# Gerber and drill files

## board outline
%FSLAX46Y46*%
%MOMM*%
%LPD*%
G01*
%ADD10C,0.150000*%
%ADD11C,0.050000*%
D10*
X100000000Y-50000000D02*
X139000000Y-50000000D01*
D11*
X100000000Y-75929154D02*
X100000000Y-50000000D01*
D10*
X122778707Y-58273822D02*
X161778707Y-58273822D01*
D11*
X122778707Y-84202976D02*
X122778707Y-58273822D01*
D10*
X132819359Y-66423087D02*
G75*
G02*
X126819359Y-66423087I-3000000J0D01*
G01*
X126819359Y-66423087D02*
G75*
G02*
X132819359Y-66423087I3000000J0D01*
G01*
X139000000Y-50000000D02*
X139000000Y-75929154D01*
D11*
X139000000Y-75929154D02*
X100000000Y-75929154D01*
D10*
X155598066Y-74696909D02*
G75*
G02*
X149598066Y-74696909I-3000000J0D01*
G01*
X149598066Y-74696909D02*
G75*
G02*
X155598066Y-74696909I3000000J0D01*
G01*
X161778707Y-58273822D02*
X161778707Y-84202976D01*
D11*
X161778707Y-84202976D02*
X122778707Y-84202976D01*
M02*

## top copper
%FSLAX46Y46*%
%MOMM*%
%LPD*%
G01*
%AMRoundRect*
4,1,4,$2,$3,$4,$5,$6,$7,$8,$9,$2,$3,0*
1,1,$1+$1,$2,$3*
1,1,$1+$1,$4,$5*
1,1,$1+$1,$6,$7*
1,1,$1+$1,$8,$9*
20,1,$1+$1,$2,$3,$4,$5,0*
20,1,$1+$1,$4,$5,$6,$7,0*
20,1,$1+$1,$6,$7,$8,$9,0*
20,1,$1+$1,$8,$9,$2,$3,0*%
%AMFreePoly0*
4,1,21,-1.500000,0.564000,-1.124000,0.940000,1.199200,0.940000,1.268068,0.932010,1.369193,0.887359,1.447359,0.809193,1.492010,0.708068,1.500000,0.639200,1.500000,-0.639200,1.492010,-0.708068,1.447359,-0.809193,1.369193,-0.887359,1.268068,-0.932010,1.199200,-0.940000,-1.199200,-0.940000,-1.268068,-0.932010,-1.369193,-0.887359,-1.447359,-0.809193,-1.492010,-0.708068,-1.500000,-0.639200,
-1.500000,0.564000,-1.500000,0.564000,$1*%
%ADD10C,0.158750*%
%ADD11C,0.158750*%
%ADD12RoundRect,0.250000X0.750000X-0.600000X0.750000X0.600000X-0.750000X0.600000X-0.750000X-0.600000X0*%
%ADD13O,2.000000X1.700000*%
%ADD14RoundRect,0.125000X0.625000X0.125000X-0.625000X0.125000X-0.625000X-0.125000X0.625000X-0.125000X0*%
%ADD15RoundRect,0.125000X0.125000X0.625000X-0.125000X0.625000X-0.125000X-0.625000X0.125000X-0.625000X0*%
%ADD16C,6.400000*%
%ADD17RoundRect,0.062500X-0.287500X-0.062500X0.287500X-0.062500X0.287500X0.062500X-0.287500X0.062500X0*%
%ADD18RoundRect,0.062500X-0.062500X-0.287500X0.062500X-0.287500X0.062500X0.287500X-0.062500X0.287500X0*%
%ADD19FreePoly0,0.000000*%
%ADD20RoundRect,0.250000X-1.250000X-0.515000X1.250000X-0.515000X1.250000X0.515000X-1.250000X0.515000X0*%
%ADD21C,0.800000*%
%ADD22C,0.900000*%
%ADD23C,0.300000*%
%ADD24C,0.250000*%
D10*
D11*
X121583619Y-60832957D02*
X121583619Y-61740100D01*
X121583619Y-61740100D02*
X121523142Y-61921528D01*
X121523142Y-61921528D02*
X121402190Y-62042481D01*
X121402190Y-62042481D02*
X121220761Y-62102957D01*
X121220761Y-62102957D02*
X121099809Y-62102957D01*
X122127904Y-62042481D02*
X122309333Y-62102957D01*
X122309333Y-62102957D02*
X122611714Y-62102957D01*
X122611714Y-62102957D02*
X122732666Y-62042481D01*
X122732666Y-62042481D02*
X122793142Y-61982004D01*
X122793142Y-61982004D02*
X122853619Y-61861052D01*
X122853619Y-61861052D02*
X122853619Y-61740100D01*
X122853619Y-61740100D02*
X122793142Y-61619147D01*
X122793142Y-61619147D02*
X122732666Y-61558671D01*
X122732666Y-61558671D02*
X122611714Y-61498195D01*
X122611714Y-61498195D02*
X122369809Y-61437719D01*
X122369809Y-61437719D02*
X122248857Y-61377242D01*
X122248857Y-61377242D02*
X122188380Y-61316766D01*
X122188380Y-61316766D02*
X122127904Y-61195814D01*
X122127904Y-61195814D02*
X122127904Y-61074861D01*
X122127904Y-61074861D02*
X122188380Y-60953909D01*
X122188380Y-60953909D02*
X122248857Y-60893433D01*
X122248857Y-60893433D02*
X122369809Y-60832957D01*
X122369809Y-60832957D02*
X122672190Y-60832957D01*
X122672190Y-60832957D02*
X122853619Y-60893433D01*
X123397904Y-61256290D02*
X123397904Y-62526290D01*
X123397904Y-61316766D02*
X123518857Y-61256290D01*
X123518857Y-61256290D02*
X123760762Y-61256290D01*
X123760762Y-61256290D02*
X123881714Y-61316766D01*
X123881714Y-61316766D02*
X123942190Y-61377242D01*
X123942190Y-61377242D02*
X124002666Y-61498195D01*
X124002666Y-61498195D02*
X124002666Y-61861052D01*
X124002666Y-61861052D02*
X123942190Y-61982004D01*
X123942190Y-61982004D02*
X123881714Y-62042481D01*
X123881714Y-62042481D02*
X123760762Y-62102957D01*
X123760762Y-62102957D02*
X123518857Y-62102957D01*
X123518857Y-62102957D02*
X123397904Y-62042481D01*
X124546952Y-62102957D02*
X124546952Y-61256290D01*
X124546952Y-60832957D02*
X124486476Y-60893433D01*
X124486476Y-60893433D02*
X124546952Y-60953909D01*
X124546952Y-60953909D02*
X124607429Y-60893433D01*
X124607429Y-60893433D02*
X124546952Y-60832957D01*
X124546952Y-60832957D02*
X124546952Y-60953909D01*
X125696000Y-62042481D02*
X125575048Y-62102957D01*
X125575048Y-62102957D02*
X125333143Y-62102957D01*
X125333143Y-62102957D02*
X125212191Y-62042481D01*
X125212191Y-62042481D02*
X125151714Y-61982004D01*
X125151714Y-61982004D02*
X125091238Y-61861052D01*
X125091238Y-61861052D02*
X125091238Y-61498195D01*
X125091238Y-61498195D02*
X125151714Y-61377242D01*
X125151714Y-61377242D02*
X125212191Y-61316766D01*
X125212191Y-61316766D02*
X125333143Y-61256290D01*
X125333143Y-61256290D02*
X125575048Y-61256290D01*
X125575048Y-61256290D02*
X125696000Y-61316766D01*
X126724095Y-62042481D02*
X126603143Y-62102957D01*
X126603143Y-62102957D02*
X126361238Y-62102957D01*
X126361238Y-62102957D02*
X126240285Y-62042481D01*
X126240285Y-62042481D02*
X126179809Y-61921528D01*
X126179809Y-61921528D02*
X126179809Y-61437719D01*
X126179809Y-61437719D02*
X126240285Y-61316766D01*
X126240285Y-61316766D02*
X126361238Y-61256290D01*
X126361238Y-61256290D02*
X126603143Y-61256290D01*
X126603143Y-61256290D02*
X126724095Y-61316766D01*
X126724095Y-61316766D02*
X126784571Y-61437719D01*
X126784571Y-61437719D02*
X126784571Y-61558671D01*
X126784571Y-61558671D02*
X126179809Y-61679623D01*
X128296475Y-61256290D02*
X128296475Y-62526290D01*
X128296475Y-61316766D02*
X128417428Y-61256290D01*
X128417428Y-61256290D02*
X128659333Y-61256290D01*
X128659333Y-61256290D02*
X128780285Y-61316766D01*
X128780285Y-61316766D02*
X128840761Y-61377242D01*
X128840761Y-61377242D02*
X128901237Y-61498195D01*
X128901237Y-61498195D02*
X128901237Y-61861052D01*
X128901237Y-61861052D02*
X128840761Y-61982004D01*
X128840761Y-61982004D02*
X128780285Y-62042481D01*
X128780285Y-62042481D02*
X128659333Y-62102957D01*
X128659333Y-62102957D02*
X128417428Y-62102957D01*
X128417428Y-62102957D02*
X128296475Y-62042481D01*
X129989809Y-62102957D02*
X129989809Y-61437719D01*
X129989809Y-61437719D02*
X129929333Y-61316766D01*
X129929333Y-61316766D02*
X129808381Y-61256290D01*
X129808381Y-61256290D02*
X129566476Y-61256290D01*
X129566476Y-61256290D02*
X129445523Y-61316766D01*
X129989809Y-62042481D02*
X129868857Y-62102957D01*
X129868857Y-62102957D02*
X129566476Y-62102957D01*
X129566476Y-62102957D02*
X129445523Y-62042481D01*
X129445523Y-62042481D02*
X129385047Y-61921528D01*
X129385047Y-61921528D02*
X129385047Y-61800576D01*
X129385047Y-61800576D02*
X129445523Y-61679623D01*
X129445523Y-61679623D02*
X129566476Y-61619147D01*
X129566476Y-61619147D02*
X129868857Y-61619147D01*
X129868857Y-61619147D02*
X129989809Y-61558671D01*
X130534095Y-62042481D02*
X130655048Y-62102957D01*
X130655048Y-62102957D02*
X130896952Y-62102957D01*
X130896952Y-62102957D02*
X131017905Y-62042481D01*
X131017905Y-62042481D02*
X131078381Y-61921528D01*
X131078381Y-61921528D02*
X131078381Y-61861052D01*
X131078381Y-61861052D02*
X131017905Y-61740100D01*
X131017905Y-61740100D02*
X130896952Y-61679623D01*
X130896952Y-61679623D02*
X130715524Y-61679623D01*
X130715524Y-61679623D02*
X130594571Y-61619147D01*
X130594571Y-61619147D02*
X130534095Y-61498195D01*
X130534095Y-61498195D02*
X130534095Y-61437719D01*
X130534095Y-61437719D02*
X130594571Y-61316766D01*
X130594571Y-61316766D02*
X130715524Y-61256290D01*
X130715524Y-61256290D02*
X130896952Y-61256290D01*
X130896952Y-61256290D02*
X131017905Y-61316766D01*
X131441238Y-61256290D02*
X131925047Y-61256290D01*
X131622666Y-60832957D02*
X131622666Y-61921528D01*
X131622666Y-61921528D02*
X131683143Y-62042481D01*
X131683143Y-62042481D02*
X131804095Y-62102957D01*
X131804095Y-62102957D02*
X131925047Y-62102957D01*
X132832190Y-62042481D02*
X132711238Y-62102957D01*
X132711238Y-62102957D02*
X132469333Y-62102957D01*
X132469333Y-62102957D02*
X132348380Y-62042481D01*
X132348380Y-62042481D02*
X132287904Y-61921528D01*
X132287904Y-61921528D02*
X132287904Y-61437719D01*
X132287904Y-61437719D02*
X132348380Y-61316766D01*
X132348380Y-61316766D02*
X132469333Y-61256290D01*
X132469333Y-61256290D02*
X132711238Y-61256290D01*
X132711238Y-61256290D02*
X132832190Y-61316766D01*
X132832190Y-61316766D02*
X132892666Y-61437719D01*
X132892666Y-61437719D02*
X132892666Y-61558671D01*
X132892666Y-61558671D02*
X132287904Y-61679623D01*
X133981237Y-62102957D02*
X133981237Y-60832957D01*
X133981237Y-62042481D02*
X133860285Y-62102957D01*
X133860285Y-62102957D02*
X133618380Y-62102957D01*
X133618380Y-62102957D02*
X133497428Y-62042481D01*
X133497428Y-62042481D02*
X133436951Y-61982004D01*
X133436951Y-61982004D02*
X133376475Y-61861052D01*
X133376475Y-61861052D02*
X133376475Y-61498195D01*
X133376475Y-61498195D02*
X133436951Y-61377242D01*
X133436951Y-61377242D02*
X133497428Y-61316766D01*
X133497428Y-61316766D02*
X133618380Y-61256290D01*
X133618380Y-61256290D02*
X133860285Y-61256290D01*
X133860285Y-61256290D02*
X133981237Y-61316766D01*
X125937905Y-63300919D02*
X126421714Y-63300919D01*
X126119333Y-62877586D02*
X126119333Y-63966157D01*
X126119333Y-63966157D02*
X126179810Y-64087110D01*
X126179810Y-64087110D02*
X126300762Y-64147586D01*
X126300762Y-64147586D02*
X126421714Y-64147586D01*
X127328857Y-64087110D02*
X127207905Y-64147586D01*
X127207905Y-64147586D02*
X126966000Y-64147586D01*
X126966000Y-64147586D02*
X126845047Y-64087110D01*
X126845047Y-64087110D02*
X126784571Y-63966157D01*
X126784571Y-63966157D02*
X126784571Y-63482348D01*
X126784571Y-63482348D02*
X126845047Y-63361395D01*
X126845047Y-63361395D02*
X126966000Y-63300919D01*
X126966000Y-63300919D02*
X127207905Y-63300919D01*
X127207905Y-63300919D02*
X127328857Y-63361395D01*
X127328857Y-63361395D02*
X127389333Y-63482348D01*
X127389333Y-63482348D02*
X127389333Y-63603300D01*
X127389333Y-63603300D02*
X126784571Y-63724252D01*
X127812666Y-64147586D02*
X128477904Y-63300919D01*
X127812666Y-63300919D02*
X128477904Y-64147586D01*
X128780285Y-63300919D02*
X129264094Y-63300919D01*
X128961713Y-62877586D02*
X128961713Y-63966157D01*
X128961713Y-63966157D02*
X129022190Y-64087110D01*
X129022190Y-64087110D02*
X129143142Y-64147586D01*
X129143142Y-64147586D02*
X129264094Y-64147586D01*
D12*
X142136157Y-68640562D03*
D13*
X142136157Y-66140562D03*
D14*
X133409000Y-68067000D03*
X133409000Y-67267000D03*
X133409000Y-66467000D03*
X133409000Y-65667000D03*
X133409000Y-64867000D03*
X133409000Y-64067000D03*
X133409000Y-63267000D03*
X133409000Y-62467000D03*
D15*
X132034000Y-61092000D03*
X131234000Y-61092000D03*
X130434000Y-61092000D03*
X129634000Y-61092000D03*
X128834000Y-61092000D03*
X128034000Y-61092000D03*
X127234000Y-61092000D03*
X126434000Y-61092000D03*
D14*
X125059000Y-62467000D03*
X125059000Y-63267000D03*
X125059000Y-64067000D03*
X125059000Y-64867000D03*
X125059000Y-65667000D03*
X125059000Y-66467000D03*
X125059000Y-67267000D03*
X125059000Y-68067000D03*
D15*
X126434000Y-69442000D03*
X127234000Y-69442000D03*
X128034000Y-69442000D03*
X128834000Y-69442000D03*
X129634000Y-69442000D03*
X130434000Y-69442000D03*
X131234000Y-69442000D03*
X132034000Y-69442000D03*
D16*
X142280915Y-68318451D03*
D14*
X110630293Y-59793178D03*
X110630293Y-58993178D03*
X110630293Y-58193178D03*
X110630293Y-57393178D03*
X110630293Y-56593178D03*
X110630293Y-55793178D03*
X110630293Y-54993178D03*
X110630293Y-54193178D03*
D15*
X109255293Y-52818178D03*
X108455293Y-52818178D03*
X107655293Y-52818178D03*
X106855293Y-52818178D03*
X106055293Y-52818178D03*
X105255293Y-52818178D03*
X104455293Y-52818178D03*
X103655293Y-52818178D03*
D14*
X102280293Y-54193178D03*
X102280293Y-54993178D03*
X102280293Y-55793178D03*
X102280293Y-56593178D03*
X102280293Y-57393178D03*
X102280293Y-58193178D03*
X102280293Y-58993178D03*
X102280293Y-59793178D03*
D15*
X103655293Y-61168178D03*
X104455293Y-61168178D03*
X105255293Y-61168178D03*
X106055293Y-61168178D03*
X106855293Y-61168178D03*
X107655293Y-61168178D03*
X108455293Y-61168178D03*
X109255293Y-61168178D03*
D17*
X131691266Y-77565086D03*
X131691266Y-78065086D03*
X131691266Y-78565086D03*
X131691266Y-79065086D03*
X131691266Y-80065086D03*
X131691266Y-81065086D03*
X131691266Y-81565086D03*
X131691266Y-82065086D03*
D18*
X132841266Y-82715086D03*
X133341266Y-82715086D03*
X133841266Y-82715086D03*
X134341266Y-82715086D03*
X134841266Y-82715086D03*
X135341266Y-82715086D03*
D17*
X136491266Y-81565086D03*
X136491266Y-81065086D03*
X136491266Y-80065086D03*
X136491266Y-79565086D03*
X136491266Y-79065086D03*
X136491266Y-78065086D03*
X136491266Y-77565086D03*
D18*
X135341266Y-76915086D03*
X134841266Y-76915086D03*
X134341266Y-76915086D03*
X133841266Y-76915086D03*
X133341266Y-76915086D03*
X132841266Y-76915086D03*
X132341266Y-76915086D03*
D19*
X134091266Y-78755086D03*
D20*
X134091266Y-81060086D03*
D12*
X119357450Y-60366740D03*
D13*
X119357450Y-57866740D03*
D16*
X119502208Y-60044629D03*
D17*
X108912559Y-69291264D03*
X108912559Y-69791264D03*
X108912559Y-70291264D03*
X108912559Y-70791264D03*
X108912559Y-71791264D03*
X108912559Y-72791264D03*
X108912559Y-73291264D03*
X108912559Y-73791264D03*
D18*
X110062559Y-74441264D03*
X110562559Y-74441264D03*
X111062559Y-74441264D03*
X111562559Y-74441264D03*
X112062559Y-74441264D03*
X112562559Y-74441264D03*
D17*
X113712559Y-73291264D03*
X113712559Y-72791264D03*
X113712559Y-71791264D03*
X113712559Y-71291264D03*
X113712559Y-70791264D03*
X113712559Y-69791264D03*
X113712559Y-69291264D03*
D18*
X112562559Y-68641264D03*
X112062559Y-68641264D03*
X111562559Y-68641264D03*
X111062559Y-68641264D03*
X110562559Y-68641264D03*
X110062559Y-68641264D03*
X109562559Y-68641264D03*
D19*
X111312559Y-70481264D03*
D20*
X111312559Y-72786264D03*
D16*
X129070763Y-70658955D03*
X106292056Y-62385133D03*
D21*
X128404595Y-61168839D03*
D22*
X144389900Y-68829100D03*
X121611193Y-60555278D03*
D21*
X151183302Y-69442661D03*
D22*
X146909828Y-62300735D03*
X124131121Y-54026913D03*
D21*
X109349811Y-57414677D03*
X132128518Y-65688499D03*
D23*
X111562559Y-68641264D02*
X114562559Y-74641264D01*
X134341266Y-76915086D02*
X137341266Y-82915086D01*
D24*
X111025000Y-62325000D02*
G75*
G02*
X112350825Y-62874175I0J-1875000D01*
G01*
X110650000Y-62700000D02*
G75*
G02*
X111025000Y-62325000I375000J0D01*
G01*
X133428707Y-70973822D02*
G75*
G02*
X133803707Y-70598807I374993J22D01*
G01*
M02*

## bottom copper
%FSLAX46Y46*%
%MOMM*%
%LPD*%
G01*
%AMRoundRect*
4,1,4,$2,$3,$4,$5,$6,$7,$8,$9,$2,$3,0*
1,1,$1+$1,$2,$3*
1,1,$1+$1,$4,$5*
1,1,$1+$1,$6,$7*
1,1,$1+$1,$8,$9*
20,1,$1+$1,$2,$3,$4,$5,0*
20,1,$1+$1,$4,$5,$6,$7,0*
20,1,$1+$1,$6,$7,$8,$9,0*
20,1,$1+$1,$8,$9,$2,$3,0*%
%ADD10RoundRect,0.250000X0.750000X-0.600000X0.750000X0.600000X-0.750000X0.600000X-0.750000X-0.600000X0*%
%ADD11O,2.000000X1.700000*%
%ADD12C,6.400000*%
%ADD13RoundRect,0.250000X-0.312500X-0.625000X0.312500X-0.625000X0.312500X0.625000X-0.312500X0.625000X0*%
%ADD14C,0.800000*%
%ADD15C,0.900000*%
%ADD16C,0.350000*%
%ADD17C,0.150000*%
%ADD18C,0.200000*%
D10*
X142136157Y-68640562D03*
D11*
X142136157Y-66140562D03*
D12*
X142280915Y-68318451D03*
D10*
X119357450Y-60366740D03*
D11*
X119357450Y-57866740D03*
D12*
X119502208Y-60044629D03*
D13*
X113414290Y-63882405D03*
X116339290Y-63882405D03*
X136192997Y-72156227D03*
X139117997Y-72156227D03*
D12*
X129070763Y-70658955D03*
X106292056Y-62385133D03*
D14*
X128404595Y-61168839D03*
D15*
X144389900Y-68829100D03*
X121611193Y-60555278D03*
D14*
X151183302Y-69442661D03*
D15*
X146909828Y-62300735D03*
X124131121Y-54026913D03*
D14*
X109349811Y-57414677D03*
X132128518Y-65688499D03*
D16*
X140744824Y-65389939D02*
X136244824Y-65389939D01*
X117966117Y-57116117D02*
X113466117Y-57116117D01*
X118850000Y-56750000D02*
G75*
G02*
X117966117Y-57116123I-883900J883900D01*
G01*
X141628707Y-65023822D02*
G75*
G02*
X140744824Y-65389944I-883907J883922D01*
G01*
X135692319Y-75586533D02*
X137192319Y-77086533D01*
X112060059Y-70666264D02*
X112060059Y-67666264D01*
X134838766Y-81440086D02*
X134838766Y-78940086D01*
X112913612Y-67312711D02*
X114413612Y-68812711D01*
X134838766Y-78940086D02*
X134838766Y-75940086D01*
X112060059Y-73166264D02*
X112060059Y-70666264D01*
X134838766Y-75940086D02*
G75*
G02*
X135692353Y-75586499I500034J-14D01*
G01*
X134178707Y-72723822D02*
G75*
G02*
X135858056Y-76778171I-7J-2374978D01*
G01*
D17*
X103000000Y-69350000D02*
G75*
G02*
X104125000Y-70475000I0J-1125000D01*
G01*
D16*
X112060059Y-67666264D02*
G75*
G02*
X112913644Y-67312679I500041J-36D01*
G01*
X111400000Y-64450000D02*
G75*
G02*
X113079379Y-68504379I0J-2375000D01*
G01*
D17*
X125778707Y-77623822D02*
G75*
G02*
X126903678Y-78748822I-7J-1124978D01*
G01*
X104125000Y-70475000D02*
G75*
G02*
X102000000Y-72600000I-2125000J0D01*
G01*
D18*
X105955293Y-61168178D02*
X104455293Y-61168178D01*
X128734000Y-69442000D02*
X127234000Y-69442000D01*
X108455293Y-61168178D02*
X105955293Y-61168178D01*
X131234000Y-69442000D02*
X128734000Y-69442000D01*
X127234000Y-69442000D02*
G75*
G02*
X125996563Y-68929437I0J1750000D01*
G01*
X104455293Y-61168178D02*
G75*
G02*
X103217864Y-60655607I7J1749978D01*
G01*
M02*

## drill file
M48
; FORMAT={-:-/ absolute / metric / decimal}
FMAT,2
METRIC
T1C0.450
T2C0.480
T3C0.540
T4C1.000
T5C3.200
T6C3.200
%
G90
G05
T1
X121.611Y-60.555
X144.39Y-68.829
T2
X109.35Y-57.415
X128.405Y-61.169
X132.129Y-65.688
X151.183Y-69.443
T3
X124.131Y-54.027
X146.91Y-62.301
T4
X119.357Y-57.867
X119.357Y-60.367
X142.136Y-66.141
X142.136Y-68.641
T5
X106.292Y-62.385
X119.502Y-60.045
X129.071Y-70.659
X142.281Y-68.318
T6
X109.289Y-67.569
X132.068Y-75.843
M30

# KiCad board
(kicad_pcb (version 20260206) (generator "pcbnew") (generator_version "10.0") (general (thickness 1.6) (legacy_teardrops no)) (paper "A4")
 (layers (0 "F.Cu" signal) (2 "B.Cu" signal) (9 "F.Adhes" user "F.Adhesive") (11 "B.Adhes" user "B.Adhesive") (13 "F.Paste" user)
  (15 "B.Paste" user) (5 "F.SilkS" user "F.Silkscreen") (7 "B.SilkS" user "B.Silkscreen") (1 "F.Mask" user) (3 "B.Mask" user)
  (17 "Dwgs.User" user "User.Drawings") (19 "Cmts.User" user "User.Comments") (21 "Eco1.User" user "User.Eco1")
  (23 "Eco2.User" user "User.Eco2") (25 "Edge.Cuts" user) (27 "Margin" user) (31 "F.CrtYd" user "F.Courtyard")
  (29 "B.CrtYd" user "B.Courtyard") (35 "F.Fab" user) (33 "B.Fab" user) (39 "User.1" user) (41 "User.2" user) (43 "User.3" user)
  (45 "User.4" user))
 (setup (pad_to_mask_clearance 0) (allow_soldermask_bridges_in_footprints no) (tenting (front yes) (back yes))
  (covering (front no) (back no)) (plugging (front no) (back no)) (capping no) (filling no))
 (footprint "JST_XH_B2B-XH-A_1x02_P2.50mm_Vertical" (layer "F.Cu") (at 142.136157 68.640562 90)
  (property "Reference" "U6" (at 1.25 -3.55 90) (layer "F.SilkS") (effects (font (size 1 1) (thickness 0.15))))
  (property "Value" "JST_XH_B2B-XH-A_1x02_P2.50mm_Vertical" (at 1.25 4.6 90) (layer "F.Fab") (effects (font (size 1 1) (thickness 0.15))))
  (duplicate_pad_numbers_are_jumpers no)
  (pad "1" thru_hole roundrect (at 0 0 90) (size 1.7 2) (drill 1) (layers "*.Cu" "*.Mask") (remove_unused_layers no)
   (roundrect_rratio 0.147059) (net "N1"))
  (pad "2" thru_hole oval (at 2.5 0 90) (size 1.7 2) (drill 1) (layers "*.Cu" "*.Mask") (remove_unused_layers no)))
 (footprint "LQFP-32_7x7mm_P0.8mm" (layer "F.Cu") (at 129.234 65.267 180)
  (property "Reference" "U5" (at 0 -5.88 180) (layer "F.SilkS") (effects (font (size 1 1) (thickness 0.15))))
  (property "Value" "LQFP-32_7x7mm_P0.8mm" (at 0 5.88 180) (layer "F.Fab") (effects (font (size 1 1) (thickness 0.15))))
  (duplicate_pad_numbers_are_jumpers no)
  (pad "1" smd roundrect (at -4.175 -2.8 180) (size 1.5 0.5) (layers "F.Cu" "F.Mask" "F.Paste") (roundrect_rratio 0.25) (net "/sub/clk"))
  (pad "2" smd roundrect (at -4.175 -2 180) (size 1.5 0.5) (layers "F.Cu" "F.Mask" "F.Paste") (roundrect_rratio 0.25) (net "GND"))
  (pad "3" smd roundrect (at -4.175 -1.2 180) (size 1.5 0.5) (layers "F.Cu" "F.Mask" "F.Paste") (roundrect_rratio 0.25) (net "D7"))
  (pad "4" smd roundrect (at -4.175 -0.4 180) (size 1.5 0.5) (layers "F.Cu" "F.Mask" "F.Paste") (roundrect_rratio 0.25) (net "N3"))
  (pad "5" smd roundrect (at -4.175 0.4 180) (size 1.5 0.5) (layers "F.Cu" "F.Mask" "F.Paste") (roundrect_rratio 0.25))
  (pad "6" smd roundrect (at -4.175 1.2 180) (size 1.5 0.5) (layers "F.Cu" "F.Mask" "F.Paste") (roundrect_rratio 0.25) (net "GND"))
  (pad "7" smd roundrect (at -4.175 2 180) (size 1.5 0.5) (layers "F.Cu" "F.Mask" "F.Paste") (roundrect_rratio 0.25))
  (pad "8" smd roundrect (at -4.175 2.8 180) (size 1.5 0.5) (layers "F.Cu" "F.Mask" "F.Paste") (roundrect_rratio 0.25) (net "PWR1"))
  (pad "9" smd roundrect (at -2.8 4.175 180) (size 0.5 1.5) (layers "F.Cu" "F.Mask" "F.Paste") (roundrect_rratio 0.25) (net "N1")
   (clearance 0.35))
  (pad "10" smd roundrect (at -2 4.175 180) (size 0.5 1.5) (layers "F.Cu" "F.Mask" "F.Paste") (roundrect_rratio 0.25) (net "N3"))
  (pad "11" smd roundrect (at -1.2 4.175 180) (size 0.5 1.5) (layers "F.Cu" "F.Mask" "F.Paste") (roundrect_rratio 0.25) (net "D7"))
  (pad "12" smd roundrect (at -0.4 4.175 180) (size 0.5 1.5) (layers "F.Cu" "F.Mask" "F.Paste") (roundrect_rratio 0.25) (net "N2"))
  (pad "13" smd roundrect (at 0.4 4.175 180) (size 0.5 1.5) (layers "F.Cu" "F.Mask" "F.Paste") (roundrect_rratio 0.25) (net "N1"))
  (pad "14" smd roundrect (at 1.2 4.175 180) (size 0.5 1.5) (layers "F.Cu" "F.Mask" "F.Paste") (roundrect_rratio 0.25) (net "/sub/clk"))
  (pad "15" smd roundrect (at 2 4.175 180) (size 0.5 1.5) (layers "F.Cu" "F.Mask" "F.Paste") (roundrect_rratio 0.25))
  (pad "16" smd roundrect (at 2.8 4.175 180) (size 0.5 1.5) (layers "F.Cu" "F.Mask" "F.Paste") (roundrect_rratio 0.25))
  (pad "17" smd roundrect (at 4.175 2.8 180) (size 1.5 0.5) (layers "F.Cu" "F.Mask" "F.Paste") (roundrect_rratio 0.25) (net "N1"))
  (pad "18" smd roundrect (at 4.175 2 180) (size 1.5 0.5) (layers "F.Cu" "F.Mask" "F.Paste") (roundrect_rratio 0.25) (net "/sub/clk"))
  (pad "19" smd roundrect (at 4.175 1.2 180) (size 1.5 0.5) (layers "F.Cu" "F.Mask" "F.Paste") (roundrect_rratio 0.25) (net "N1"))
  (pad "20" smd roundrect (at 4.175 0.4 180) (size 1.5 0.5) (layers "F.Cu" "F.Mask" "F.Paste") (roundrect_rratio 0.25) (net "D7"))
  (pad "21" smd roundrect (at 4.175 -0.4 180) (size 1.5 0.5) (layers "F.Cu" "F.Mask" "F.Paste") (roundrect_rratio 0.25) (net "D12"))
  (pad "22" smd roundrect (at 4.175 -1.2 180) (size 1.5 0.5) (layers "F.Cu" "F.Mask" "F.Paste") (roundrect_rratio 0.25))
  (pad "23" smd roundrect (at 4.175 -2 180) (size 1.5 0.5) (layers "F.Cu" "F.Mask" "F.Paste") (roundrect_rratio 0.25))
  (pad "24" smd roundrect (at 4.175 -2.8 180) (size 1.5 0.5) (layers "F.Cu" "F.Mask" "F.Paste") (roundrect_rratio 0.25))
  (pad "25" smd roundrect (at 2.8 -4.175 180) (size 0.5 1.5) (layers "F.Cu" "F.Mask" "F.Paste") (roundrect_rratio 0.25) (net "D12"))
  (pad "26" smd roundrect (at 2 -4.175 180) (size 0.5 1.5) (layers "F.Cu" "F.Mask" "F.Paste") (roundrect_rratio 0.25) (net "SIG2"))
  (pad "27" smd roundrect (at 1.2 -4.175 180) (size 0.5 1.5) (layers "F.Cu" "F.Mask" "F.Paste") (roundrect_rratio 0.25) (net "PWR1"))
  (pad "28" smd roundrect (at 0.4 -4.175 180) (size 0.5 1.5) (layers "F.Cu" "F.Mask" "F.Paste") (roundrect_rratio 0.25) (clearance 0.35))
  (pad "29" smd roundrect (at -0.4 -4.175 180) (size 0.5 1.5) (layers "F.Cu" "F.Mask" "F.Paste") (roundrect_rratio 0.25) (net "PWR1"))
  (pad "30" smd roundrect (at -1.2 -4.175 180) (size 0.5 1.5) (layers "F.Cu" "F.Mask" "F.Paste") (roundrect_rratio 0.25) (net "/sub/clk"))
  (pad "31" smd roundrect (at -2 -4.175 180) (size 0.5 1.5) (layers "F.Cu" "F.Mask" "F.Paste") (roundrect_rratio 0.25) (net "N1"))
  (pad "32" smd roundrect (at -2.8 -4.175 180) (size 0.5 1.5) (layers "F.Cu" "F.Mask" "F.Paste") (roundrect_rratio 0.25) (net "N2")))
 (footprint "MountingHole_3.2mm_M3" (layer "F.Cu") (at 109.289246 67.568769)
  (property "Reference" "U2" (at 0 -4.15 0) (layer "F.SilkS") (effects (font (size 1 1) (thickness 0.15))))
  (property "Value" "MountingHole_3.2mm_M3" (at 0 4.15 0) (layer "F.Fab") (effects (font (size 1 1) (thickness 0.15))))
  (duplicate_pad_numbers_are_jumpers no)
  (pad "" np_thru_hole circle (at 0 0) (size 3.2 3.2) (drill 3.2) (layers "*.Cu" "*.Mask")))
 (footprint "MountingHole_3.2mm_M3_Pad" (layer "F.Cu") (at 142.280915 68.318451)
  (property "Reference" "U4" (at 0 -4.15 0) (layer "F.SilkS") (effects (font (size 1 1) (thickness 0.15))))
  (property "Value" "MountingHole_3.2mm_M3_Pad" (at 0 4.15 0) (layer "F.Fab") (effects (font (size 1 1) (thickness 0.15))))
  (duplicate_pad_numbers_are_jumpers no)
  (pad "1" thru_hole circle (at 0 0) (size 6.4 6.4) (drill 3.2) (layers "*.Cu" "*.Mask") (remove_unused_layers no) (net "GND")
   (zone_connect 2)))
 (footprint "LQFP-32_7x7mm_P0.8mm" (layer "F.Cu") (at 106.455293 56.993178 180)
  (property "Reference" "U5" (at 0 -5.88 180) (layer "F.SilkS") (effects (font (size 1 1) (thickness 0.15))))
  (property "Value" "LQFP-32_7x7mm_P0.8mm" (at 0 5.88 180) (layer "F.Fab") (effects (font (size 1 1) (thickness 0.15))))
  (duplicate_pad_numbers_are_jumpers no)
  (pad "1" smd roundrect (at -4.175 -2.8 180) (size 1.5 0.5) (layers "F.Cu" "F.Mask" "F.Paste") (roundrect_rratio 0.25) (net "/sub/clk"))
  (pad "2" smd roundrect (at -4.175 -2 180) (size 1.5 0.5) (layers "F.Cu" "F.Mask" "F.Paste") (roundrect_rratio 0.25) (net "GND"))
  (pad "3" smd roundrect (at -4.175 -1.2 180) (size 1.5 0.5) (layers "F.Cu" "F.Mask" "F.Paste") (roundrect_rratio 0.25) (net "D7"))
  (pad "4" smd roundrect (at -4.175 -0.4 180) (size 1.5 0.5) (layers "F.Cu" "F.Mask" "F.Paste") (roundrect_rratio 0.25) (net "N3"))
  (pad "5" smd roundrect (at -4.175 0.4 180) (size 1.5 0.5) (layers "F.Cu" "F.Mask" "F.Paste") (roundrect_rratio 0.25))
  (pad "6" smd roundrect (at -4.175 1.2 180) (size 1.5 0.5) (layers "F.Cu" "F.Mask" "F.Paste") (roundrect_rratio 0.25) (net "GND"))
  (pad "7" smd roundrect (at -4.175 2 180) (size 1.5 0.5) (layers "F.Cu" "F.Mask" "F.Paste") (roundrect_rratio 0.25))
  (pad "8" smd roundrect (at -4.175 2.8 180) (size 1.5 0.5) (layers "F.Cu" "F.Mask" "F.Paste") (roundrect_rratio 0.25) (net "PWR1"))
  (pad "9" smd roundrect (at -2.8 4.175 180) (size 0.5 1.5) (layers "F.Cu" "F.Mask" "F.Paste") (roundrect_rratio 0.25) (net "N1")
   (clearance 0.35))
  (pad "10" smd roundrect (at -2 4.175 180) (size 0.5 1.5) (layers "F.Cu" "F.Mask" "F.Paste") (roundrect_rratio 0.25) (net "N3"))
  (pad "11" smd roundrect (at -1.2 4.175 180) (size 0.5 1.5) (layers "F.Cu" "F.Mask" "F.Paste") (roundrect_rratio 0.25) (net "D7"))
  (pad "12" smd roundrect (at -0.4 4.175 180) (size 0.5 1.5) (layers "F.Cu" "F.Mask" "F.Paste") (roundrect_rratio 0.25) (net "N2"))
  (pad "13" smd roundrect (at 0.4 4.175 180) (size 0.5 1.5) (layers "F.Cu" "F.Mask" "F.Paste") (roundrect_rratio 0.25) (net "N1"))
  (pad "14" smd roundrect (at 1.2 4.175 180) (size 0.5 1.5) (layers "F.Cu" "F.Mask" "F.Paste") (roundrect_rratio 0.25) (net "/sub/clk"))
  (pad "15" smd roundrect (at 2 4.175 180) (size 0.5 1.5) (layers "F.Cu" "F.Mask" "F.Paste") (roundrect_rratio 0.25))
  (pad "16" smd roundrect (at 2.8 4.175 180) (size 0.5 1.5) (layers "F.Cu" "F.Mask" "F.Paste") (roundrect_rratio 0.25))
  (pad "17" smd roundrect (at 4.175 2.8 180) (size 1.5 0.5) (layers "F.Cu" "F.Mask" "F.Paste") (roundrect_rratio 0.25) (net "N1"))
  (pad "18" smd roundrect (at 4.175 2 180) (size 1.5 0.5) (layers "F.Cu" "F.Mask" "F.Paste") (roundrect_rratio 0.25) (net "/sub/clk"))
  (pad "19" smd roundrect (at 4.175 1.2 180) (size 1.5 0.5) (layers "F.Cu" "F.Mask" "F.Paste") (roundrect_rratio 0.25) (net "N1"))
  (pad "20" smd roundrect (at 4.175 0.4 180) (size 1.5 0.5) (layers "F.Cu" "F.Mask" "F.Paste") (roundrect_rratio 0.25) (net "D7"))
  (pad "21" smd roundrect (at 4.175 -0.4 180) (size 1.5 0.5) (layers "F.Cu" "F.Mask" "F.Paste") (roundrect_rratio 0.25) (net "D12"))
  (pad "22" smd roundrect (at 4.175 -1.2 180) (size 1.5 0.5) (layers "F.Cu" "F.Mask" "F.Paste") (roundrect_rratio 0.25))
  (pad "23" smd roundrect (at 4.175 -2 180) (size 1.5 0.5) (layers "F.Cu" "F.Mask" "F.Paste") (roundrect_rratio 0.25))
  (pad "24" smd roundrect (at 4.175 -2.8 180) (size 1.5 0.5) (layers "F.Cu" "F.Mask" "F.Paste") (roundrect_rratio 0.25))
  (pad "25" smd roundrect (at 2.8 -4.175 180) (size 0.5 1.5) (layers "F.Cu" "F.Mask" "F.Paste") (roundrect_rratio 0.25) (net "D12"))
  (pad "26" smd roundrect (at 2 -4.175 180) (size 0.5 1.5) (layers "F.Cu" "F.Mask" "F.Paste") (roundrect_rratio 0.25) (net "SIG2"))
  (pad "27" smd roundrect (at 1.2 -4.175 180) (size 0.5 1.5) (layers "F.Cu" "F.Mask" "F.Paste") (roundrect_rratio 0.25) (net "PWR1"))
  (pad "28" smd roundrect (at 0.4 -4.175 180) (size 0.5 1.5) (layers "F.Cu" "F.Mask" "F.Paste") (roundrect_rratio 0.25) (clearance 0.35))
  (pad "29" smd roundrect (at -0.4 -4.175 180) (size 0.5 1.5) (layers "F.Cu" "F.Mask" "F.Paste") (roundrect_rratio 0.25) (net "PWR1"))
  (pad "30" smd roundrect (at -1.2 -4.175 180) (size 0.5 1.5) (layers "F.Cu" "F.Mask" "F.Paste") (roundrect_rratio 0.25) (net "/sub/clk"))
  (pad "31" smd roundrect (at -2 -4.175 180) (size 0.5 1.5) (layers "F.Cu" "F.Mask" "F.Paste") (roundrect_rratio 0.25) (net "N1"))
  (pad "32" smd roundrect (at -2.8 -4.175 180) (size 0.5 1.5) (layers "F.Cu" "F.Mask" "F.Paste") (roundrect_rratio 0.25) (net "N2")))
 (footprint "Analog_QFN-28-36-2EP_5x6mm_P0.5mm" (layer "F.Cu") (at 134.091266 79.815086)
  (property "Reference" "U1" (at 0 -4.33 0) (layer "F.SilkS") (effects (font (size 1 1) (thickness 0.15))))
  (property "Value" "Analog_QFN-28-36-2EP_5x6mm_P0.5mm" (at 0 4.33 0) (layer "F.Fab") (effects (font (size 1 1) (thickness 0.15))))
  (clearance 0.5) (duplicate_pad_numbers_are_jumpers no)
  (pad "" smd roundrect (at -0.75 -1.53) (size 1.21 0.76) (layers "F.Paste") (roundrect_rratio 0.25) (chamfer_ratio 0.4) (chamfer top_left)
   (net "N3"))
  (pad "" smd roundrect (at -0.75 -0.59) (size 1.21 0.76) (layers "F.Paste") (roundrect_rratio 0.25) (clearance 0.1))
  (pad "" smd roundrect (at -0.7475 0.875) (size 1.205 0.55) (layers "F.Paste") (roundrect_rratio 0.25) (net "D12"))
  (pad "" smd roundrect (at -0.7475 1.625) (size 1.205 0.55) (layers "F.Paste") (roundrect_rratio 0.25) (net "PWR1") (clearance 0.35))
  (pad "" smd roundrect (at 0.7475 0.875) (size 1.205 0.55) (layers "F.Paste") (roundrect_rratio 0.25) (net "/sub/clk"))
  (pad "" smd roundrect (at 0.7475 1.625) (size 1.205 0.55) (layers "F.Paste") (roundrect_rratio 0.25) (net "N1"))
  (pad "" smd roundrect (at 0.75 -1.53) (size 1.21 0.76) (layers "F.Paste") (roundrect_rratio 0.25) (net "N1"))
  (pad "" smd roundrect (at 0.75 -0.59) (size 1.21 0.76) (layers "F.Paste") (roundrect_rratio 0.25) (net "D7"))
  (pad "1" smd roundrect (at -2.4 -2.25) (size 0.7 0.25) (layers "F.Cu" "F.Mask" "F.Paste") (roundrect_rratio 0.25) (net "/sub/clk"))
  (pad "2" smd roundrect (at -2.4 -1.75) (size 0.7 0.25) (layers "F.Cu" "F.Mask" "F.Paste") (roundrect_rratio 0.25) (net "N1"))
  (pad "3" smd roundrect (at -2.4 -1.25) (size 0.7 0.25) (layers "F.Cu" "F.Mask" "F.Paste") (roundrect_rratio 0.25))
  (pad "4" smd roundrect (at -2.4 -0.75) (size 0.7 0.25) (layers "F.Cu" "F.Mask" "F.Paste") (roundrect_rratio 0.25))
  (pad "6" smd roundrect (at -2.4 0.25) (size 0.7 0.25) (layers "F.Cu" "F.Mask" "F.Paste") (roundrect_rratio 0.25) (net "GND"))
  (pad "8" smd roundrect (at -2.4 1.25) (size 0.7 0.25) (layers "F.Cu" "F.Mask" "F.Paste") (roundrect_rratio 0.25))
  (pad "9" smd roundrect (at -2.4 1.75) (size 0.7 0.25) (layers "F.Cu" "F.Mask" "F.Paste") (roundrect_rratio 0.25) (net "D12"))
  (pad "10" smd roundrect (at -2.4 2.25) (size 0.7 0.25) (layers "F.Cu" "F.Mask" "F.Paste") (roundrect_rratio 0.25) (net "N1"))
  (pad "12" smd roundrect (at -1.25 2.9) (size 0.25 0.7) (layers "F.Cu" "F.Mask" "F.Paste") (roundrect_rratio 0.25))
  (pad "13" smd roundrect (at -0.75 2.9) (size 0.25 0.7) (layers "F.Cu" "F.Mask" "F.Paste") (roundrect_rratio 0.25) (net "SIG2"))
  (pad "14" smd roundrect (at -0.25 2.9) (size 0.25 0.7) (layers "F.Cu" "F.Mask" "F.Paste") (roundrect_rratio 0.25) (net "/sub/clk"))
  (pad "15" smd roundrect (at 0.25 2.9) (size 0.25 0.7) (layers "F.Cu" "F.Mask" "F.Paste") (roundrect_rratio 0.25))
  (pad "16" smd roundrect (at 0.75 2.9) (size 0.25 0.7) (layers "F.Cu" "F.Mask" "F.Paste") (roundrect_rratio 0.25) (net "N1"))
  (pad "17" smd roundrect (at 1.25 2.9) (size 0.25 0.7) (layers "F.Cu" "F.Mask" "F.Paste") (roundrect_rratio 0.25) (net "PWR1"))
  (pad "20" smd roundrect (at 2.4 1.75) (size 0.7 0.25) (layers "F.Cu" "F.Mask" "F.Paste") (roundrect_rratio 0.25) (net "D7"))
  (pad "21" smd roundrect (at 2.4 1.25) (size 0.7 0.25) (layers "F.Cu" "F.Mask" "F.Paste") (roundrect_rratio 0.25) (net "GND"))
  (pad "23" smd roundrect (at 2.4 0.25) (size 0.7 0.25) (layers "F.Cu" "F.Mask" "F.Paste") (roundrect_rratio 0.25))
  (pad "24" smd roundrect (at 2.4 -0.25) (size 0.7 0.25) (layers "F.Cu" "F.Mask" "F.Paste") (roundrect_rratio 0.25) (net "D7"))
  (pad "25" smd roundrect (at 2.4 -0.75) (size 0.7 0.25) (layers "F.Cu" "F.Mask" "F.Paste") (roundrect_rratio 0.25) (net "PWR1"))
  (pad "27" smd roundrect (at 2.4 -1.75) (size 0.7 0.25) (layers "F.Cu" "F.Mask" "F.Paste") (roundrect_rratio 0.25) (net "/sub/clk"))
  (pad "28" smd roundrect (at 2.4 -2.25) (size 0.7 0.25) (layers "F.Cu" "F.Mask" "F.Paste") (roundrect_rratio 0.25) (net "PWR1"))
  (pad "30" smd roundrect (at 1.25 -2.9) (size 0.25 0.7) (layers "F.Cu" "F.Mask" "F.Paste") (roundrect_rratio 0.25))
  (pad "31" smd roundrect (at 0.75 -2.9) (size 0.25 0.7) (layers "F.Cu" "F.Mask" "F.Paste") (roundrect_rratio 0.25))
  (pad "32" smd roundrect (at 0.25 -2.9) (size 0.25 0.7) (layers "F.Cu" "F.Mask" "F.Paste") (roundrect_rratio 0.25))
  (pad "33" smd roundrect (at -0.25 -2.9) (size 0.25 0.7) (layers "F.Cu" "F.Mask" "F.Paste") (roundrect_rratio 0.25) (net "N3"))
  (pad "34" smd roundrect (at -0.75 -2.9) (size 0.25 0.7) (layers "F.Cu" "F.Mask" "F.Paste") (roundrect_rratio 0.25))
  (pad "35" smd roundrect (at -1.25 -2.9) (size 0.25 0.7) (layers "F.Cu" "F.Mask" "F.Paste") (roundrect_rratio 0.25))
  (pad "36" smd roundrect (at -1.75 -2.9) (size 0.25 0.7) (layers "F.Cu" "F.Mask" "F.Paste") (roundrect_rratio 0.25) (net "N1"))
  (pad "37" smd roundrect (at 0 -1.06) (size 3 1.88) (layers "F.Cu" "F.Mask") (roundrect_rratio 0.16) (chamfer_ratio 0.2) (chamfer top_left)
   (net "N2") (zone_connect 2))
  (pad "38" smd roundrect (at 0 1.245) (size 3 1.53) (layers "F.Cu" "F.Mask") (roundrect_rratio 0.1633986928) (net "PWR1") (zone_connect 2)))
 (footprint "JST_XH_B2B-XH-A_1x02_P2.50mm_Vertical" (layer "F.Cu") (at 119.35745 60.36674 90)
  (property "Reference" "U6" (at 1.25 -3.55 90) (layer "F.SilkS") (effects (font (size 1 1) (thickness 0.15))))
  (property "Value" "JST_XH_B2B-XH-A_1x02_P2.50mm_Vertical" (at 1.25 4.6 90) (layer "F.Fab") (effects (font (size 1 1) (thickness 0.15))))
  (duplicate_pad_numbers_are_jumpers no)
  (pad "1" thru_hole roundrect (at 0 0 90) (size 1.7 2) (drill 1) (layers "*.Cu" "*.Mask") (remove_unused_layers no)
   (roundrect_rratio 0.147059) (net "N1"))
  (pad "2" thru_hole oval (at 2.5 0 90) (size 1.7 2) (drill 1) (layers "*.Cu" "*.Mask") (remove_unused_layers no)))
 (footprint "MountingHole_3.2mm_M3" (layer "F.Cu") (at 132.067953 75.842591)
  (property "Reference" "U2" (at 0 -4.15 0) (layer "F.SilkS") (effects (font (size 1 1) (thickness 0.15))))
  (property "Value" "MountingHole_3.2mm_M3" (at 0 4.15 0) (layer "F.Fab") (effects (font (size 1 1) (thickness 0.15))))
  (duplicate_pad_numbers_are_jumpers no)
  (pad "" np_thru_hole circle (at 0 0) (size 3.2 3.2) (drill 3.2) (layers "*.Cu" "*.Mask")))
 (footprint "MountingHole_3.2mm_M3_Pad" (layer "F.Cu") (at 119.502208 60.044629)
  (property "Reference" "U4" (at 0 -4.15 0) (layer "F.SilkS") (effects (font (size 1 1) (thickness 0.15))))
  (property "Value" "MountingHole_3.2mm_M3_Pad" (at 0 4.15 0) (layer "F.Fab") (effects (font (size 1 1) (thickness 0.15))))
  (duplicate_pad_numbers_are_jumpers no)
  (pad "1" thru_hole circle (at 0 0) (size 6.4 6.4) (drill 3.2) (layers "*.Cu" "*.Mask") (remove_unused_layers no) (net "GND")
   (zone_connect 2)))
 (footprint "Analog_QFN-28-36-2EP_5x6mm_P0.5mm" (layer "F.Cu") (at 111.312559 71.541264)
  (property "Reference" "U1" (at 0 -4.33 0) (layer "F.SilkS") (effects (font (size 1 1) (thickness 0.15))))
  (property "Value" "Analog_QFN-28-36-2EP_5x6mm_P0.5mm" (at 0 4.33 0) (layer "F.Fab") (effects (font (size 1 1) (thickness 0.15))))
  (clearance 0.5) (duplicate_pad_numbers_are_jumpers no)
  (pad "" smd roundrect (at -0.75 -1.53) (size 1.21 0.76) (layers "F.Paste") (roundrect_rratio 0.25) (chamfer_ratio 0.4) (chamfer top_left)
   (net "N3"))
  (pad "" smd roundrect (at -0.75 -0.59) (size 1.21 0.76) (layers "F.Paste") (roundrect_rratio 0.25) (clearance 0.1))
  (pad "" smd roundrect (at -0.7475 0.875) (size 1.205 0.55) (layers "F.Paste") (roundrect_rratio 0.25) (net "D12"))
  (pad "" smd roundrect (at -0.7475 1.625) (size 1.205 0.55) (layers "F.Paste") (roundrect_rratio 0.25) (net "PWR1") (clearance 0.35))
  (pad "" smd roundrect (at 0.7475 0.875) (size 1.205 0.55) (layers "F.Paste") (roundrect_rratio 0.25) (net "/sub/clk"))
  (pad "" smd roundrect (at 0.7475 1.625) (size 1.205 0.55) (layers "F.Paste") (roundrect_rratio 0.25) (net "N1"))
  (pad "" smd roundrect (at 0.75 -1.53) (size 1.21 0.76) (layers "F.Paste") (roundrect_rratio 0.25) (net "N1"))
  (pad "" smd roundrect (at 0.75 -0.59) (size 1.21 0.76) (layers "F.Paste") (roundrect_rratio 0.25) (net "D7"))
  (pad "1" smd roundrect (at -2.4 -2.25) (size 0.7 0.25) (layers "F.Cu" "F.Mask" "F.Paste") (roundrect_rratio 0.25) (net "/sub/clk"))
  (pad "2" smd roundrect (at -2.4 -1.75) (size 0.7 0.25) (layers "F.Cu" "F.Mask" "F.Paste") (roundrect_rratio 0.25) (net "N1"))
  (pad "3" smd roundrect (at -2.4 -1.25) (size 0.7 0.25) (layers "F.Cu" "F.Mask" "F.Paste") (roundrect_rratio 0.25))
  (pad "4" smd roundrect (at -2.4 -0.75) (size 0.7 0.25) (layers "F.Cu" "F.Mask" "F.Paste") (roundrect_rratio 0.25))
  (pad "6" smd roundrect (at -2.4 0.25) (size 0.7 0.25) (layers "F.Cu" "F.Mask" "F.Paste") (roundrect_rratio 0.25) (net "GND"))
  (pad "8" smd roundrect (at -2.4 1.25) (size 0.7 0.25) (layers "F.Cu" "F.Mask" "F.Paste") (roundrect_rratio 0.25))
  (pad "9" smd roundrect (at -2.4 1.75) (size 0.7 0.25) (layers "F.Cu" "F.Mask" "F.Paste") (roundrect_rratio 0.25) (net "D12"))
  (pad "10" smd roundrect (at -2.4 2.25) (size 0.7 0.25) (layers "F.Cu" "F.Mask" "F.Paste") (roundrect_rratio 0.25) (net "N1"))
  (pad "12" smd roundrect (at -1.25 2.9) (size 0.25 0.7) (layers "F.Cu" "F.Mask" "F.Paste") (roundrect_rratio 0.25))
  (pad "13" smd roundrect (at -0.75 2.9) (size 0.25 0.7) (layers "F.Cu" "F.Mask" "F.Paste") (roundrect_rratio 0.25) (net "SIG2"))
  (pad "14" smd roundrect (at -0.25 2.9) (size 0.25 0.7) (layers "F.Cu" "F.Mask" "F.Paste") (roundrect_rratio 0.25) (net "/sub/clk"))
  (pad "15" smd roundrect (at 0.25 2.9) (size 0.25 0.7) (layers "F.Cu" "F.Mask" "F.Paste") (roundrect_rratio 0.25))
  (pad "16" smd roundrect (at 0.75 2.9) (size 0.25 0.7) (layers "F.Cu" "F.Mask" "F.Paste") (roundrect_rratio 0.25) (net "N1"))
  (pad "17" smd roundrect (at 1.25 2.9) (size 0.25 0.7) (layers "F.Cu" "F.Mask" "F.Paste") (roundrect_rratio 0.25) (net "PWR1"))
  (pad "20" smd roundrect (at 2.4 1.75) (size 0.7 0.25) (layers "F.Cu" "F.Mask" "F.Paste") (roundrect_rratio 0.25) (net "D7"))
  (pad "21" smd roundrect (at 2.4 1.25) (size 0.7 0.25) (layers "F.Cu" "F.Mask" "F.Paste") (roundrect_rratio 0.25) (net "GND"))
  (pad "23" smd roundrect (at 2.4 0.25) (size 0.7 0.25) (layers "F.Cu" "F.Mask" "F.Paste") (roundrect_rratio 0.25))
  (pad "24" smd roundrect (at 2.4 -0.25) (size 0.7 0.25) (layers "F.Cu" "F.Mask" "F.Paste") (roundrect_rratio 0.25) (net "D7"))
  (pad "25" smd roundrect (at 2.4 -0.75) (size 0.7 0.25) (layers "F.Cu" "F.Mask" "F.Paste") (roundrect_rratio 0.25) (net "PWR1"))
  (pad "27" smd roundrect (at 2.4 -1.75) (size 0.7 0.25) (layers "F.Cu" "F.Mask" "F.Paste") (roundrect_rratio 0.25) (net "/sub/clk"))
  (pad "28" smd roundrect (at 2.4 -2.25) (size 0.7 0.25) (layers "F.Cu" "F.Mask" "F.Paste") (roundrect_rratio 0.25) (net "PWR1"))
  (pad "30" smd roundrect (at 1.25 -2.9) (size 0.25 0.7) (layers "F.Cu" "F.Mask" "F.Paste") (roundrect_rratio 0.25))
  (pad "31" smd roundrect (at 0.75 -2.9) (size 0.25 0.7) (layers "F.Cu" "F.Mask" "F.Paste") (roundrect_rratio 0.25))
  (pad "32" smd roundrect (at 0.25 -2.9) (size 0.25 0.7) (layers "F.Cu" "F.Mask" "F.Paste") (roundrect_rratio 0.25))
  (pad "33" smd roundrect (at -0.25 -2.9) (size 0.25 0.7) (layers "F.Cu" "F.Mask" "F.Paste") (roundrect_rratio 0.25) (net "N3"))
  (pad "34" smd roundrect (at -0.75 -2.9) (size 0.25 0.7) (layers "F.Cu" "F.Mask" "F.Paste") (roundrect_rratio 0.25))
  (pad "35" smd roundrect (at -1.25 -2.9) (size 0.25 0.7) (layers "F.Cu" "F.Mask" "F.Paste") (roundrect_rratio 0.25))
  (pad "36" smd roundrect (at -1.75 -2.9) (size 0.25 0.7) (layers "F.Cu" "F.Mask" "F.Paste") (roundrect_rratio 0.25) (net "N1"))
  (pad "37" smd roundrect (at 0 -1.06) (size 3 1.88) (layers "F.Cu" "F.Mask") (roundrect_rratio 0.16) (chamfer_ratio 0.2) (chamfer top_left)
   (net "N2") (zone_connect 2))
  (pad "38" smd roundrect (at 0 1.245) (size 3 1.53) (layers "F.Cu" "F.Mask") (roundrect_rratio 0.1633986928) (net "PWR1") (zone_connect 2)))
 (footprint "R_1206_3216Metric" (layer "B.Cu") (at 114.87679 63.882405)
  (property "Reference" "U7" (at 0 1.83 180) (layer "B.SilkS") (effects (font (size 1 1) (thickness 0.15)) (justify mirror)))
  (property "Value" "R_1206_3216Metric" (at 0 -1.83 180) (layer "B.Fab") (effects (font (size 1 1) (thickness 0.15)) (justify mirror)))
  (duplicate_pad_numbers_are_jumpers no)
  (pad "1" smd roundrect (at -1.4625 0) (size 1.125 1.75) (layers "B.Cu" "B.Mask" "B.Paste") (roundrect_rratio 0.222222) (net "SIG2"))
  (pad "2" smd roundrect (at 1.4625 0) (size 1.125 1.75) (layers "B.Cu" "B.Mask" "B.Paste") (roundrect_rratio 0.222222) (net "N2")))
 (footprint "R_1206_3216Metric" (layer "B.Cu") (at 137.655497 72.156227)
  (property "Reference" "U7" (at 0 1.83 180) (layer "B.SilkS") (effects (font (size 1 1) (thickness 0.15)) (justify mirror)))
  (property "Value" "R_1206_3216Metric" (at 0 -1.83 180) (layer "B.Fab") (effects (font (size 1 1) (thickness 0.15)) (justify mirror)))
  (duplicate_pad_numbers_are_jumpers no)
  (pad "1" smd roundrect (at -1.4625 0) (size 1.125 1.75) (layers "B.Cu" "B.Mask" "B.Paste") (roundrect_rratio 0.222222) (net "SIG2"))
  (pad "2" smd roundrect (at 1.4625 0) (size 1.125 1.75) (layers "B.Cu" "B.Mask" "B.Paste") (roundrect_rratio 0.222222) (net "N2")))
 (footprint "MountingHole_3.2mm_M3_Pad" (layer "B.Cu") (at 129.070763 70.658955 90)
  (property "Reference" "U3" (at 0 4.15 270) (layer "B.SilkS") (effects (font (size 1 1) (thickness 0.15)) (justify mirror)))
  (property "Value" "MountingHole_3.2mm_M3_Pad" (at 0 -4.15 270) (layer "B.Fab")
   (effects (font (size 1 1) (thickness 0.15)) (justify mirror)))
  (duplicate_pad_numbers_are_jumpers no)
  (pad "1" thru_hole circle (at 0 0 90) (size 6.4 6.4) (drill 3.2) (layers "*.Cu" "*.Mask") (remove_unused_layers no) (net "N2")
   (clearance 0.1) (zone_connect 2)))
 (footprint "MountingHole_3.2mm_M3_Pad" (layer "B.Cu") (at 106.292056 62.385133 90)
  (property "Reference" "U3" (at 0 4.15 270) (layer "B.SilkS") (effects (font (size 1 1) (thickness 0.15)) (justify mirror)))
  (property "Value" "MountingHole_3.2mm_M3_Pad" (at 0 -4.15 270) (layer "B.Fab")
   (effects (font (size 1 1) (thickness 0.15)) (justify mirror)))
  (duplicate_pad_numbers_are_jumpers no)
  (pad "1" thru_hole circle (at 0 0 90) (size 6.4 6.4) (drill 3.2) (layers "*.Cu" "*.Mask") (remove_unused_layers no) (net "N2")
   (clearance 0.1) (zone_connect 2)))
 (gr_line (start 100 50) (end 139 50) (stroke (width 0.15) (type default)) (layer "Edge.Cuts"))
 (gr_line (start 100 75.929154) (end 100 50) (stroke (width 0.05) (type default)) (layer "Edge.Cuts"))
 (gr_line (start 122.778707 58.273822) (end 161.778707 58.273822) (stroke (width 0.15) (type default)) (layer "Edge.Cuts"))
 (gr_line (start 122.778707 84.202976) (end 122.778707 58.273822) (stroke (width 0.05) (type default)) (layer "Edge.Cuts"))
 (gr_circle (center 129.819359 66.423087) (end 132.819359 66.423087) (stroke (width 0.15) (type default)) (fill no) (layer "Edge.Cuts"))
 (gr_line (start 139 50) (end 139 75.929154) (stroke (width 0.15) (type default)) (layer "Edge.Cuts"))
 (gr_line (start 139 75.929154) (end 100 75.929154) (stroke (width 0.05) (type default)) (layer "Edge.Cuts"))
 (gr_circle (center 152.598066 74.696909) (end 155.598066 74.696909) (stroke (width 0.15) (type default)) (fill no) (layer "Edge.Cuts"))
 (gr_line (start 161.778707 58.273822) (end 161.778707 84.202976) (stroke (width 0.15) (type default)) (layer "Edge.Cuts"))
 (gr_line (start 161.778707 84.202976) (end 122.778707 84.202976) (stroke (width 0.05) (type default)) (layer "Edge.Cuts"))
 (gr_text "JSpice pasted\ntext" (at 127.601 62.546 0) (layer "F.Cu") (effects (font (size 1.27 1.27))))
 (segment (start 111.562559 68.641264) (end 114.562559 74.641264) (width 0.3) (layer "F.Cu") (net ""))
 (segment (start 134.341266 76.915086) (end 137.341266 82.915086) (width 0.3) (layer "F.Cu") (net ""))
 (arc (start 111.025 62.325) (mid 111.742531 62.467726) (end 112.350825 62.874175) (width 0.25) (locked yes) (layer "F.Cu") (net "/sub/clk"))
 (arc (start 110.65 62.7) (mid 110.759835 62.434835) (end 111.025 62.325) (width 0.25) (layer "F.Cu") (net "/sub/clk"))
 (arc (start 133.428707 70.973822) (mid 133.538542 70.708657) (end 133.803707 70.598822) (width 0.25) (layer "F.Cu") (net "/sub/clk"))
 (via (at 128.404595 61.168839) (size 0.8) (drill 0.48) (layers "F.Cu" "B.Cu") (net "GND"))
 (via (at 144.3899 68.8291) (size 0.9) (drill 0.45) (layers "F.Cu" "B.Cu") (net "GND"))
 (via (at 121.611193 60.555278) (size 0.9) (drill 0.45) (layers "F.Cu" "B.Cu") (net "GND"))
 (via (at 151.183302 69.442661) (size 0.8) (drill 0.48) (layers "F.Cu" "B.Cu") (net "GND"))
 (segment (start 140.744824 65.389939) (end 136.244824 65.389939) (width 0.35) (layer "B.Cu") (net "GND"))
 (segment (start 117.966117 57.116117) (end 113.466117 57.116117) (width 0.35) (layer "B.Cu") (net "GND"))
 (arc (start 118.85 56.75) (mid 118.444471 57.020966) (end 117.966117 57.116117) (width 0.35) (layer "B.Cu") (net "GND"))
 (arc (start 141.628707 65.023822) (mid 141.223178 65.294788) (end 140.744824 65.389939) (width 0.35) (layer "B.Cu") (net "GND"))
 (via (at 146.909828 62.300735) (size 0.9) (drill 0.54) (layers "F.Cu" "B.Cu") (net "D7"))
 (via (at 124.131121 54.026913) (size 0.9) (drill 0.54) (layers "F.Cu" "B.Cu") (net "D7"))
 (via (at 109.349811 57.414677) (size 0.8) (drill 0.48) (layers "F.Cu" "B.Cu") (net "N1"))
 (via (at 132.128518 65.688499) (size 0.8) (drill 0.48) (layers "F.Cu" "B.Cu") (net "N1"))
 (segment (start 135.692319 75.586533) (end 137.192319 77.086533) (width 0.35) (layer "B.Cu") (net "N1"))
 (segment (start 112.060059 70.666264) (end 112.060059 67.666264) (width 0.35) (layer "B.Cu") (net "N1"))
 (segment (start 134.838766 81.440086) (end 134.838766 78.940086) (width 0.35) (layer "B.Cu") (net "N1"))
 (segment (start 112.913612 67.312711) (end 114.413612 68.812711) (width 0.35) (layer "B.Cu") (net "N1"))
 (segment (start 134.838766 78.940086) (end 134.838766 75.940086) (width 0.35) (layer "B.Cu") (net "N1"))
 (segment (start 112.060059 73.166264) (end 112.060059 70.666264) (width 0.35) (layer "B.Cu") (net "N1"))
 (arc (start 134.838766 75.940086) (mid 135.147424 75.478146) (end 135.692319 75.586533) (width 0.35) (layer "B.Cu") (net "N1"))
 (arc (start 134.178707 72.723822) (mid 136.372921 74.189949) (end 135.858086 76.778201) (width 0.35) (layer "B.Cu") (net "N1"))
 (arc (start 103 69.35) (mid 103.795495 69.679505) (end 104.125 70.475) (width 0.15) (layer "B.Cu") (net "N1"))
 (arc (start 112.060059 67.666264) (mid 112.368717 67.204324) (end 112.913612 67.312711) (width 0.35) (layer "B.Cu") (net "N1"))
 (arc (start 111.4 64.45) (mid 113.594214 65.916127) (end 113.079379 68.504379) (width 0.35) (layer "B.Cu") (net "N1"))
 (arc (start 125.778707 77.623822) (mid 126.574202 77.953327) (end 126.903707 78.748822) (width 0.15) (layer "B.Cu") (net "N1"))
 (arc (start 104.125 70.475) (mid 103.502602 71.977602) (end 102 72.6) (width 0.15) (locked yes) (layer "B.Cu") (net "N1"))
 (segment (start 105.955293 61.168178) (end 104.455293 61.168178) (width 0.2) (layer "B.Cu") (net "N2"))
 (segment (start 128.734 69.442) (end 127.234 69.442) (width 0.2) (layer "B.Cu") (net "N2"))
 (segment (start 108.455293 61.168178) (end 105.955293 61.168178) (width 0.2) (layer "B.Cu") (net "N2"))
 (segment (start 131.234 69.442) (end 128.734 69.442) (width 0.2) (layer "B.Cu") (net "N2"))
 (arc (start 127.234 69.442) (mid 126.564304 69.308789) (end 125.996563 68.929437) (width 0.2) (layer "B.Cu") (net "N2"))
 (arc (start 104.455293 61.168178) (mid 103.785597 61.034967) (end 103.217856 60.655615) (width 0.2) (layer "B.Cu") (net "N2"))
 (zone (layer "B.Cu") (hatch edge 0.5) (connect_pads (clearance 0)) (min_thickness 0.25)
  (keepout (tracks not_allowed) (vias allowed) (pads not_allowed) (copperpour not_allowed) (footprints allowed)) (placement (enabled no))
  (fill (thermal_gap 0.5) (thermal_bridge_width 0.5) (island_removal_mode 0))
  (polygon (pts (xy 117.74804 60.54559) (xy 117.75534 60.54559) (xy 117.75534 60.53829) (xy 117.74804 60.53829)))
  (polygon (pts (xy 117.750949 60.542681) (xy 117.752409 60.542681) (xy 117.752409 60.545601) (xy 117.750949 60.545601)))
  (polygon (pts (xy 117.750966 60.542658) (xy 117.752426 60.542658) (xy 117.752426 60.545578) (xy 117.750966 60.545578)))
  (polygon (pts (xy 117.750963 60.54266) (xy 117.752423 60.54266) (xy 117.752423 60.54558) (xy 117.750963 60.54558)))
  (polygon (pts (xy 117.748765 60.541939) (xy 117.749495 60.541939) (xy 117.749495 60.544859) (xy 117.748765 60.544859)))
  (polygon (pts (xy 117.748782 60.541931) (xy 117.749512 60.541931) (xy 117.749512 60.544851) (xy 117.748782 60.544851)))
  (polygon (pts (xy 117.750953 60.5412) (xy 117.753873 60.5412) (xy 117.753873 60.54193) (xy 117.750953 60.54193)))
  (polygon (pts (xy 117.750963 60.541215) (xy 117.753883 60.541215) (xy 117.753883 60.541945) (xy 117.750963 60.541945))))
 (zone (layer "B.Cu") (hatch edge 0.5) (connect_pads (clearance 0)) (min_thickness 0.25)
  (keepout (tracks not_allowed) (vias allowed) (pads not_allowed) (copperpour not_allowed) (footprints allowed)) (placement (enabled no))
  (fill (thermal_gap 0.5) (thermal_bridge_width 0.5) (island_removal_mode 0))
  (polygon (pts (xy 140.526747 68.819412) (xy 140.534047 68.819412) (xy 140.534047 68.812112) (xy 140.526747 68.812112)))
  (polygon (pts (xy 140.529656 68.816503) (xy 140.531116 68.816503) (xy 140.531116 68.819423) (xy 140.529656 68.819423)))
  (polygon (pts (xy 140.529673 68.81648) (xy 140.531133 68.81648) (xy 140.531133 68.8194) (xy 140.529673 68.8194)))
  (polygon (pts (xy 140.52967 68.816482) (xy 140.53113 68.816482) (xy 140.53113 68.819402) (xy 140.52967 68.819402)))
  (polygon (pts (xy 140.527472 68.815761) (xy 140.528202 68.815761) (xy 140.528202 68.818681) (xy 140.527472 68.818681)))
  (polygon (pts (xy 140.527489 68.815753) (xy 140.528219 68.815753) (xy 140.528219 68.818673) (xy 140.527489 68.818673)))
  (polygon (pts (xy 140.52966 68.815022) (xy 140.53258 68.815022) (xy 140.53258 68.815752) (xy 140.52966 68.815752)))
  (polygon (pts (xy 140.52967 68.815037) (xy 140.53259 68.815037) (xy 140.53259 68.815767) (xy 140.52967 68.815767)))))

